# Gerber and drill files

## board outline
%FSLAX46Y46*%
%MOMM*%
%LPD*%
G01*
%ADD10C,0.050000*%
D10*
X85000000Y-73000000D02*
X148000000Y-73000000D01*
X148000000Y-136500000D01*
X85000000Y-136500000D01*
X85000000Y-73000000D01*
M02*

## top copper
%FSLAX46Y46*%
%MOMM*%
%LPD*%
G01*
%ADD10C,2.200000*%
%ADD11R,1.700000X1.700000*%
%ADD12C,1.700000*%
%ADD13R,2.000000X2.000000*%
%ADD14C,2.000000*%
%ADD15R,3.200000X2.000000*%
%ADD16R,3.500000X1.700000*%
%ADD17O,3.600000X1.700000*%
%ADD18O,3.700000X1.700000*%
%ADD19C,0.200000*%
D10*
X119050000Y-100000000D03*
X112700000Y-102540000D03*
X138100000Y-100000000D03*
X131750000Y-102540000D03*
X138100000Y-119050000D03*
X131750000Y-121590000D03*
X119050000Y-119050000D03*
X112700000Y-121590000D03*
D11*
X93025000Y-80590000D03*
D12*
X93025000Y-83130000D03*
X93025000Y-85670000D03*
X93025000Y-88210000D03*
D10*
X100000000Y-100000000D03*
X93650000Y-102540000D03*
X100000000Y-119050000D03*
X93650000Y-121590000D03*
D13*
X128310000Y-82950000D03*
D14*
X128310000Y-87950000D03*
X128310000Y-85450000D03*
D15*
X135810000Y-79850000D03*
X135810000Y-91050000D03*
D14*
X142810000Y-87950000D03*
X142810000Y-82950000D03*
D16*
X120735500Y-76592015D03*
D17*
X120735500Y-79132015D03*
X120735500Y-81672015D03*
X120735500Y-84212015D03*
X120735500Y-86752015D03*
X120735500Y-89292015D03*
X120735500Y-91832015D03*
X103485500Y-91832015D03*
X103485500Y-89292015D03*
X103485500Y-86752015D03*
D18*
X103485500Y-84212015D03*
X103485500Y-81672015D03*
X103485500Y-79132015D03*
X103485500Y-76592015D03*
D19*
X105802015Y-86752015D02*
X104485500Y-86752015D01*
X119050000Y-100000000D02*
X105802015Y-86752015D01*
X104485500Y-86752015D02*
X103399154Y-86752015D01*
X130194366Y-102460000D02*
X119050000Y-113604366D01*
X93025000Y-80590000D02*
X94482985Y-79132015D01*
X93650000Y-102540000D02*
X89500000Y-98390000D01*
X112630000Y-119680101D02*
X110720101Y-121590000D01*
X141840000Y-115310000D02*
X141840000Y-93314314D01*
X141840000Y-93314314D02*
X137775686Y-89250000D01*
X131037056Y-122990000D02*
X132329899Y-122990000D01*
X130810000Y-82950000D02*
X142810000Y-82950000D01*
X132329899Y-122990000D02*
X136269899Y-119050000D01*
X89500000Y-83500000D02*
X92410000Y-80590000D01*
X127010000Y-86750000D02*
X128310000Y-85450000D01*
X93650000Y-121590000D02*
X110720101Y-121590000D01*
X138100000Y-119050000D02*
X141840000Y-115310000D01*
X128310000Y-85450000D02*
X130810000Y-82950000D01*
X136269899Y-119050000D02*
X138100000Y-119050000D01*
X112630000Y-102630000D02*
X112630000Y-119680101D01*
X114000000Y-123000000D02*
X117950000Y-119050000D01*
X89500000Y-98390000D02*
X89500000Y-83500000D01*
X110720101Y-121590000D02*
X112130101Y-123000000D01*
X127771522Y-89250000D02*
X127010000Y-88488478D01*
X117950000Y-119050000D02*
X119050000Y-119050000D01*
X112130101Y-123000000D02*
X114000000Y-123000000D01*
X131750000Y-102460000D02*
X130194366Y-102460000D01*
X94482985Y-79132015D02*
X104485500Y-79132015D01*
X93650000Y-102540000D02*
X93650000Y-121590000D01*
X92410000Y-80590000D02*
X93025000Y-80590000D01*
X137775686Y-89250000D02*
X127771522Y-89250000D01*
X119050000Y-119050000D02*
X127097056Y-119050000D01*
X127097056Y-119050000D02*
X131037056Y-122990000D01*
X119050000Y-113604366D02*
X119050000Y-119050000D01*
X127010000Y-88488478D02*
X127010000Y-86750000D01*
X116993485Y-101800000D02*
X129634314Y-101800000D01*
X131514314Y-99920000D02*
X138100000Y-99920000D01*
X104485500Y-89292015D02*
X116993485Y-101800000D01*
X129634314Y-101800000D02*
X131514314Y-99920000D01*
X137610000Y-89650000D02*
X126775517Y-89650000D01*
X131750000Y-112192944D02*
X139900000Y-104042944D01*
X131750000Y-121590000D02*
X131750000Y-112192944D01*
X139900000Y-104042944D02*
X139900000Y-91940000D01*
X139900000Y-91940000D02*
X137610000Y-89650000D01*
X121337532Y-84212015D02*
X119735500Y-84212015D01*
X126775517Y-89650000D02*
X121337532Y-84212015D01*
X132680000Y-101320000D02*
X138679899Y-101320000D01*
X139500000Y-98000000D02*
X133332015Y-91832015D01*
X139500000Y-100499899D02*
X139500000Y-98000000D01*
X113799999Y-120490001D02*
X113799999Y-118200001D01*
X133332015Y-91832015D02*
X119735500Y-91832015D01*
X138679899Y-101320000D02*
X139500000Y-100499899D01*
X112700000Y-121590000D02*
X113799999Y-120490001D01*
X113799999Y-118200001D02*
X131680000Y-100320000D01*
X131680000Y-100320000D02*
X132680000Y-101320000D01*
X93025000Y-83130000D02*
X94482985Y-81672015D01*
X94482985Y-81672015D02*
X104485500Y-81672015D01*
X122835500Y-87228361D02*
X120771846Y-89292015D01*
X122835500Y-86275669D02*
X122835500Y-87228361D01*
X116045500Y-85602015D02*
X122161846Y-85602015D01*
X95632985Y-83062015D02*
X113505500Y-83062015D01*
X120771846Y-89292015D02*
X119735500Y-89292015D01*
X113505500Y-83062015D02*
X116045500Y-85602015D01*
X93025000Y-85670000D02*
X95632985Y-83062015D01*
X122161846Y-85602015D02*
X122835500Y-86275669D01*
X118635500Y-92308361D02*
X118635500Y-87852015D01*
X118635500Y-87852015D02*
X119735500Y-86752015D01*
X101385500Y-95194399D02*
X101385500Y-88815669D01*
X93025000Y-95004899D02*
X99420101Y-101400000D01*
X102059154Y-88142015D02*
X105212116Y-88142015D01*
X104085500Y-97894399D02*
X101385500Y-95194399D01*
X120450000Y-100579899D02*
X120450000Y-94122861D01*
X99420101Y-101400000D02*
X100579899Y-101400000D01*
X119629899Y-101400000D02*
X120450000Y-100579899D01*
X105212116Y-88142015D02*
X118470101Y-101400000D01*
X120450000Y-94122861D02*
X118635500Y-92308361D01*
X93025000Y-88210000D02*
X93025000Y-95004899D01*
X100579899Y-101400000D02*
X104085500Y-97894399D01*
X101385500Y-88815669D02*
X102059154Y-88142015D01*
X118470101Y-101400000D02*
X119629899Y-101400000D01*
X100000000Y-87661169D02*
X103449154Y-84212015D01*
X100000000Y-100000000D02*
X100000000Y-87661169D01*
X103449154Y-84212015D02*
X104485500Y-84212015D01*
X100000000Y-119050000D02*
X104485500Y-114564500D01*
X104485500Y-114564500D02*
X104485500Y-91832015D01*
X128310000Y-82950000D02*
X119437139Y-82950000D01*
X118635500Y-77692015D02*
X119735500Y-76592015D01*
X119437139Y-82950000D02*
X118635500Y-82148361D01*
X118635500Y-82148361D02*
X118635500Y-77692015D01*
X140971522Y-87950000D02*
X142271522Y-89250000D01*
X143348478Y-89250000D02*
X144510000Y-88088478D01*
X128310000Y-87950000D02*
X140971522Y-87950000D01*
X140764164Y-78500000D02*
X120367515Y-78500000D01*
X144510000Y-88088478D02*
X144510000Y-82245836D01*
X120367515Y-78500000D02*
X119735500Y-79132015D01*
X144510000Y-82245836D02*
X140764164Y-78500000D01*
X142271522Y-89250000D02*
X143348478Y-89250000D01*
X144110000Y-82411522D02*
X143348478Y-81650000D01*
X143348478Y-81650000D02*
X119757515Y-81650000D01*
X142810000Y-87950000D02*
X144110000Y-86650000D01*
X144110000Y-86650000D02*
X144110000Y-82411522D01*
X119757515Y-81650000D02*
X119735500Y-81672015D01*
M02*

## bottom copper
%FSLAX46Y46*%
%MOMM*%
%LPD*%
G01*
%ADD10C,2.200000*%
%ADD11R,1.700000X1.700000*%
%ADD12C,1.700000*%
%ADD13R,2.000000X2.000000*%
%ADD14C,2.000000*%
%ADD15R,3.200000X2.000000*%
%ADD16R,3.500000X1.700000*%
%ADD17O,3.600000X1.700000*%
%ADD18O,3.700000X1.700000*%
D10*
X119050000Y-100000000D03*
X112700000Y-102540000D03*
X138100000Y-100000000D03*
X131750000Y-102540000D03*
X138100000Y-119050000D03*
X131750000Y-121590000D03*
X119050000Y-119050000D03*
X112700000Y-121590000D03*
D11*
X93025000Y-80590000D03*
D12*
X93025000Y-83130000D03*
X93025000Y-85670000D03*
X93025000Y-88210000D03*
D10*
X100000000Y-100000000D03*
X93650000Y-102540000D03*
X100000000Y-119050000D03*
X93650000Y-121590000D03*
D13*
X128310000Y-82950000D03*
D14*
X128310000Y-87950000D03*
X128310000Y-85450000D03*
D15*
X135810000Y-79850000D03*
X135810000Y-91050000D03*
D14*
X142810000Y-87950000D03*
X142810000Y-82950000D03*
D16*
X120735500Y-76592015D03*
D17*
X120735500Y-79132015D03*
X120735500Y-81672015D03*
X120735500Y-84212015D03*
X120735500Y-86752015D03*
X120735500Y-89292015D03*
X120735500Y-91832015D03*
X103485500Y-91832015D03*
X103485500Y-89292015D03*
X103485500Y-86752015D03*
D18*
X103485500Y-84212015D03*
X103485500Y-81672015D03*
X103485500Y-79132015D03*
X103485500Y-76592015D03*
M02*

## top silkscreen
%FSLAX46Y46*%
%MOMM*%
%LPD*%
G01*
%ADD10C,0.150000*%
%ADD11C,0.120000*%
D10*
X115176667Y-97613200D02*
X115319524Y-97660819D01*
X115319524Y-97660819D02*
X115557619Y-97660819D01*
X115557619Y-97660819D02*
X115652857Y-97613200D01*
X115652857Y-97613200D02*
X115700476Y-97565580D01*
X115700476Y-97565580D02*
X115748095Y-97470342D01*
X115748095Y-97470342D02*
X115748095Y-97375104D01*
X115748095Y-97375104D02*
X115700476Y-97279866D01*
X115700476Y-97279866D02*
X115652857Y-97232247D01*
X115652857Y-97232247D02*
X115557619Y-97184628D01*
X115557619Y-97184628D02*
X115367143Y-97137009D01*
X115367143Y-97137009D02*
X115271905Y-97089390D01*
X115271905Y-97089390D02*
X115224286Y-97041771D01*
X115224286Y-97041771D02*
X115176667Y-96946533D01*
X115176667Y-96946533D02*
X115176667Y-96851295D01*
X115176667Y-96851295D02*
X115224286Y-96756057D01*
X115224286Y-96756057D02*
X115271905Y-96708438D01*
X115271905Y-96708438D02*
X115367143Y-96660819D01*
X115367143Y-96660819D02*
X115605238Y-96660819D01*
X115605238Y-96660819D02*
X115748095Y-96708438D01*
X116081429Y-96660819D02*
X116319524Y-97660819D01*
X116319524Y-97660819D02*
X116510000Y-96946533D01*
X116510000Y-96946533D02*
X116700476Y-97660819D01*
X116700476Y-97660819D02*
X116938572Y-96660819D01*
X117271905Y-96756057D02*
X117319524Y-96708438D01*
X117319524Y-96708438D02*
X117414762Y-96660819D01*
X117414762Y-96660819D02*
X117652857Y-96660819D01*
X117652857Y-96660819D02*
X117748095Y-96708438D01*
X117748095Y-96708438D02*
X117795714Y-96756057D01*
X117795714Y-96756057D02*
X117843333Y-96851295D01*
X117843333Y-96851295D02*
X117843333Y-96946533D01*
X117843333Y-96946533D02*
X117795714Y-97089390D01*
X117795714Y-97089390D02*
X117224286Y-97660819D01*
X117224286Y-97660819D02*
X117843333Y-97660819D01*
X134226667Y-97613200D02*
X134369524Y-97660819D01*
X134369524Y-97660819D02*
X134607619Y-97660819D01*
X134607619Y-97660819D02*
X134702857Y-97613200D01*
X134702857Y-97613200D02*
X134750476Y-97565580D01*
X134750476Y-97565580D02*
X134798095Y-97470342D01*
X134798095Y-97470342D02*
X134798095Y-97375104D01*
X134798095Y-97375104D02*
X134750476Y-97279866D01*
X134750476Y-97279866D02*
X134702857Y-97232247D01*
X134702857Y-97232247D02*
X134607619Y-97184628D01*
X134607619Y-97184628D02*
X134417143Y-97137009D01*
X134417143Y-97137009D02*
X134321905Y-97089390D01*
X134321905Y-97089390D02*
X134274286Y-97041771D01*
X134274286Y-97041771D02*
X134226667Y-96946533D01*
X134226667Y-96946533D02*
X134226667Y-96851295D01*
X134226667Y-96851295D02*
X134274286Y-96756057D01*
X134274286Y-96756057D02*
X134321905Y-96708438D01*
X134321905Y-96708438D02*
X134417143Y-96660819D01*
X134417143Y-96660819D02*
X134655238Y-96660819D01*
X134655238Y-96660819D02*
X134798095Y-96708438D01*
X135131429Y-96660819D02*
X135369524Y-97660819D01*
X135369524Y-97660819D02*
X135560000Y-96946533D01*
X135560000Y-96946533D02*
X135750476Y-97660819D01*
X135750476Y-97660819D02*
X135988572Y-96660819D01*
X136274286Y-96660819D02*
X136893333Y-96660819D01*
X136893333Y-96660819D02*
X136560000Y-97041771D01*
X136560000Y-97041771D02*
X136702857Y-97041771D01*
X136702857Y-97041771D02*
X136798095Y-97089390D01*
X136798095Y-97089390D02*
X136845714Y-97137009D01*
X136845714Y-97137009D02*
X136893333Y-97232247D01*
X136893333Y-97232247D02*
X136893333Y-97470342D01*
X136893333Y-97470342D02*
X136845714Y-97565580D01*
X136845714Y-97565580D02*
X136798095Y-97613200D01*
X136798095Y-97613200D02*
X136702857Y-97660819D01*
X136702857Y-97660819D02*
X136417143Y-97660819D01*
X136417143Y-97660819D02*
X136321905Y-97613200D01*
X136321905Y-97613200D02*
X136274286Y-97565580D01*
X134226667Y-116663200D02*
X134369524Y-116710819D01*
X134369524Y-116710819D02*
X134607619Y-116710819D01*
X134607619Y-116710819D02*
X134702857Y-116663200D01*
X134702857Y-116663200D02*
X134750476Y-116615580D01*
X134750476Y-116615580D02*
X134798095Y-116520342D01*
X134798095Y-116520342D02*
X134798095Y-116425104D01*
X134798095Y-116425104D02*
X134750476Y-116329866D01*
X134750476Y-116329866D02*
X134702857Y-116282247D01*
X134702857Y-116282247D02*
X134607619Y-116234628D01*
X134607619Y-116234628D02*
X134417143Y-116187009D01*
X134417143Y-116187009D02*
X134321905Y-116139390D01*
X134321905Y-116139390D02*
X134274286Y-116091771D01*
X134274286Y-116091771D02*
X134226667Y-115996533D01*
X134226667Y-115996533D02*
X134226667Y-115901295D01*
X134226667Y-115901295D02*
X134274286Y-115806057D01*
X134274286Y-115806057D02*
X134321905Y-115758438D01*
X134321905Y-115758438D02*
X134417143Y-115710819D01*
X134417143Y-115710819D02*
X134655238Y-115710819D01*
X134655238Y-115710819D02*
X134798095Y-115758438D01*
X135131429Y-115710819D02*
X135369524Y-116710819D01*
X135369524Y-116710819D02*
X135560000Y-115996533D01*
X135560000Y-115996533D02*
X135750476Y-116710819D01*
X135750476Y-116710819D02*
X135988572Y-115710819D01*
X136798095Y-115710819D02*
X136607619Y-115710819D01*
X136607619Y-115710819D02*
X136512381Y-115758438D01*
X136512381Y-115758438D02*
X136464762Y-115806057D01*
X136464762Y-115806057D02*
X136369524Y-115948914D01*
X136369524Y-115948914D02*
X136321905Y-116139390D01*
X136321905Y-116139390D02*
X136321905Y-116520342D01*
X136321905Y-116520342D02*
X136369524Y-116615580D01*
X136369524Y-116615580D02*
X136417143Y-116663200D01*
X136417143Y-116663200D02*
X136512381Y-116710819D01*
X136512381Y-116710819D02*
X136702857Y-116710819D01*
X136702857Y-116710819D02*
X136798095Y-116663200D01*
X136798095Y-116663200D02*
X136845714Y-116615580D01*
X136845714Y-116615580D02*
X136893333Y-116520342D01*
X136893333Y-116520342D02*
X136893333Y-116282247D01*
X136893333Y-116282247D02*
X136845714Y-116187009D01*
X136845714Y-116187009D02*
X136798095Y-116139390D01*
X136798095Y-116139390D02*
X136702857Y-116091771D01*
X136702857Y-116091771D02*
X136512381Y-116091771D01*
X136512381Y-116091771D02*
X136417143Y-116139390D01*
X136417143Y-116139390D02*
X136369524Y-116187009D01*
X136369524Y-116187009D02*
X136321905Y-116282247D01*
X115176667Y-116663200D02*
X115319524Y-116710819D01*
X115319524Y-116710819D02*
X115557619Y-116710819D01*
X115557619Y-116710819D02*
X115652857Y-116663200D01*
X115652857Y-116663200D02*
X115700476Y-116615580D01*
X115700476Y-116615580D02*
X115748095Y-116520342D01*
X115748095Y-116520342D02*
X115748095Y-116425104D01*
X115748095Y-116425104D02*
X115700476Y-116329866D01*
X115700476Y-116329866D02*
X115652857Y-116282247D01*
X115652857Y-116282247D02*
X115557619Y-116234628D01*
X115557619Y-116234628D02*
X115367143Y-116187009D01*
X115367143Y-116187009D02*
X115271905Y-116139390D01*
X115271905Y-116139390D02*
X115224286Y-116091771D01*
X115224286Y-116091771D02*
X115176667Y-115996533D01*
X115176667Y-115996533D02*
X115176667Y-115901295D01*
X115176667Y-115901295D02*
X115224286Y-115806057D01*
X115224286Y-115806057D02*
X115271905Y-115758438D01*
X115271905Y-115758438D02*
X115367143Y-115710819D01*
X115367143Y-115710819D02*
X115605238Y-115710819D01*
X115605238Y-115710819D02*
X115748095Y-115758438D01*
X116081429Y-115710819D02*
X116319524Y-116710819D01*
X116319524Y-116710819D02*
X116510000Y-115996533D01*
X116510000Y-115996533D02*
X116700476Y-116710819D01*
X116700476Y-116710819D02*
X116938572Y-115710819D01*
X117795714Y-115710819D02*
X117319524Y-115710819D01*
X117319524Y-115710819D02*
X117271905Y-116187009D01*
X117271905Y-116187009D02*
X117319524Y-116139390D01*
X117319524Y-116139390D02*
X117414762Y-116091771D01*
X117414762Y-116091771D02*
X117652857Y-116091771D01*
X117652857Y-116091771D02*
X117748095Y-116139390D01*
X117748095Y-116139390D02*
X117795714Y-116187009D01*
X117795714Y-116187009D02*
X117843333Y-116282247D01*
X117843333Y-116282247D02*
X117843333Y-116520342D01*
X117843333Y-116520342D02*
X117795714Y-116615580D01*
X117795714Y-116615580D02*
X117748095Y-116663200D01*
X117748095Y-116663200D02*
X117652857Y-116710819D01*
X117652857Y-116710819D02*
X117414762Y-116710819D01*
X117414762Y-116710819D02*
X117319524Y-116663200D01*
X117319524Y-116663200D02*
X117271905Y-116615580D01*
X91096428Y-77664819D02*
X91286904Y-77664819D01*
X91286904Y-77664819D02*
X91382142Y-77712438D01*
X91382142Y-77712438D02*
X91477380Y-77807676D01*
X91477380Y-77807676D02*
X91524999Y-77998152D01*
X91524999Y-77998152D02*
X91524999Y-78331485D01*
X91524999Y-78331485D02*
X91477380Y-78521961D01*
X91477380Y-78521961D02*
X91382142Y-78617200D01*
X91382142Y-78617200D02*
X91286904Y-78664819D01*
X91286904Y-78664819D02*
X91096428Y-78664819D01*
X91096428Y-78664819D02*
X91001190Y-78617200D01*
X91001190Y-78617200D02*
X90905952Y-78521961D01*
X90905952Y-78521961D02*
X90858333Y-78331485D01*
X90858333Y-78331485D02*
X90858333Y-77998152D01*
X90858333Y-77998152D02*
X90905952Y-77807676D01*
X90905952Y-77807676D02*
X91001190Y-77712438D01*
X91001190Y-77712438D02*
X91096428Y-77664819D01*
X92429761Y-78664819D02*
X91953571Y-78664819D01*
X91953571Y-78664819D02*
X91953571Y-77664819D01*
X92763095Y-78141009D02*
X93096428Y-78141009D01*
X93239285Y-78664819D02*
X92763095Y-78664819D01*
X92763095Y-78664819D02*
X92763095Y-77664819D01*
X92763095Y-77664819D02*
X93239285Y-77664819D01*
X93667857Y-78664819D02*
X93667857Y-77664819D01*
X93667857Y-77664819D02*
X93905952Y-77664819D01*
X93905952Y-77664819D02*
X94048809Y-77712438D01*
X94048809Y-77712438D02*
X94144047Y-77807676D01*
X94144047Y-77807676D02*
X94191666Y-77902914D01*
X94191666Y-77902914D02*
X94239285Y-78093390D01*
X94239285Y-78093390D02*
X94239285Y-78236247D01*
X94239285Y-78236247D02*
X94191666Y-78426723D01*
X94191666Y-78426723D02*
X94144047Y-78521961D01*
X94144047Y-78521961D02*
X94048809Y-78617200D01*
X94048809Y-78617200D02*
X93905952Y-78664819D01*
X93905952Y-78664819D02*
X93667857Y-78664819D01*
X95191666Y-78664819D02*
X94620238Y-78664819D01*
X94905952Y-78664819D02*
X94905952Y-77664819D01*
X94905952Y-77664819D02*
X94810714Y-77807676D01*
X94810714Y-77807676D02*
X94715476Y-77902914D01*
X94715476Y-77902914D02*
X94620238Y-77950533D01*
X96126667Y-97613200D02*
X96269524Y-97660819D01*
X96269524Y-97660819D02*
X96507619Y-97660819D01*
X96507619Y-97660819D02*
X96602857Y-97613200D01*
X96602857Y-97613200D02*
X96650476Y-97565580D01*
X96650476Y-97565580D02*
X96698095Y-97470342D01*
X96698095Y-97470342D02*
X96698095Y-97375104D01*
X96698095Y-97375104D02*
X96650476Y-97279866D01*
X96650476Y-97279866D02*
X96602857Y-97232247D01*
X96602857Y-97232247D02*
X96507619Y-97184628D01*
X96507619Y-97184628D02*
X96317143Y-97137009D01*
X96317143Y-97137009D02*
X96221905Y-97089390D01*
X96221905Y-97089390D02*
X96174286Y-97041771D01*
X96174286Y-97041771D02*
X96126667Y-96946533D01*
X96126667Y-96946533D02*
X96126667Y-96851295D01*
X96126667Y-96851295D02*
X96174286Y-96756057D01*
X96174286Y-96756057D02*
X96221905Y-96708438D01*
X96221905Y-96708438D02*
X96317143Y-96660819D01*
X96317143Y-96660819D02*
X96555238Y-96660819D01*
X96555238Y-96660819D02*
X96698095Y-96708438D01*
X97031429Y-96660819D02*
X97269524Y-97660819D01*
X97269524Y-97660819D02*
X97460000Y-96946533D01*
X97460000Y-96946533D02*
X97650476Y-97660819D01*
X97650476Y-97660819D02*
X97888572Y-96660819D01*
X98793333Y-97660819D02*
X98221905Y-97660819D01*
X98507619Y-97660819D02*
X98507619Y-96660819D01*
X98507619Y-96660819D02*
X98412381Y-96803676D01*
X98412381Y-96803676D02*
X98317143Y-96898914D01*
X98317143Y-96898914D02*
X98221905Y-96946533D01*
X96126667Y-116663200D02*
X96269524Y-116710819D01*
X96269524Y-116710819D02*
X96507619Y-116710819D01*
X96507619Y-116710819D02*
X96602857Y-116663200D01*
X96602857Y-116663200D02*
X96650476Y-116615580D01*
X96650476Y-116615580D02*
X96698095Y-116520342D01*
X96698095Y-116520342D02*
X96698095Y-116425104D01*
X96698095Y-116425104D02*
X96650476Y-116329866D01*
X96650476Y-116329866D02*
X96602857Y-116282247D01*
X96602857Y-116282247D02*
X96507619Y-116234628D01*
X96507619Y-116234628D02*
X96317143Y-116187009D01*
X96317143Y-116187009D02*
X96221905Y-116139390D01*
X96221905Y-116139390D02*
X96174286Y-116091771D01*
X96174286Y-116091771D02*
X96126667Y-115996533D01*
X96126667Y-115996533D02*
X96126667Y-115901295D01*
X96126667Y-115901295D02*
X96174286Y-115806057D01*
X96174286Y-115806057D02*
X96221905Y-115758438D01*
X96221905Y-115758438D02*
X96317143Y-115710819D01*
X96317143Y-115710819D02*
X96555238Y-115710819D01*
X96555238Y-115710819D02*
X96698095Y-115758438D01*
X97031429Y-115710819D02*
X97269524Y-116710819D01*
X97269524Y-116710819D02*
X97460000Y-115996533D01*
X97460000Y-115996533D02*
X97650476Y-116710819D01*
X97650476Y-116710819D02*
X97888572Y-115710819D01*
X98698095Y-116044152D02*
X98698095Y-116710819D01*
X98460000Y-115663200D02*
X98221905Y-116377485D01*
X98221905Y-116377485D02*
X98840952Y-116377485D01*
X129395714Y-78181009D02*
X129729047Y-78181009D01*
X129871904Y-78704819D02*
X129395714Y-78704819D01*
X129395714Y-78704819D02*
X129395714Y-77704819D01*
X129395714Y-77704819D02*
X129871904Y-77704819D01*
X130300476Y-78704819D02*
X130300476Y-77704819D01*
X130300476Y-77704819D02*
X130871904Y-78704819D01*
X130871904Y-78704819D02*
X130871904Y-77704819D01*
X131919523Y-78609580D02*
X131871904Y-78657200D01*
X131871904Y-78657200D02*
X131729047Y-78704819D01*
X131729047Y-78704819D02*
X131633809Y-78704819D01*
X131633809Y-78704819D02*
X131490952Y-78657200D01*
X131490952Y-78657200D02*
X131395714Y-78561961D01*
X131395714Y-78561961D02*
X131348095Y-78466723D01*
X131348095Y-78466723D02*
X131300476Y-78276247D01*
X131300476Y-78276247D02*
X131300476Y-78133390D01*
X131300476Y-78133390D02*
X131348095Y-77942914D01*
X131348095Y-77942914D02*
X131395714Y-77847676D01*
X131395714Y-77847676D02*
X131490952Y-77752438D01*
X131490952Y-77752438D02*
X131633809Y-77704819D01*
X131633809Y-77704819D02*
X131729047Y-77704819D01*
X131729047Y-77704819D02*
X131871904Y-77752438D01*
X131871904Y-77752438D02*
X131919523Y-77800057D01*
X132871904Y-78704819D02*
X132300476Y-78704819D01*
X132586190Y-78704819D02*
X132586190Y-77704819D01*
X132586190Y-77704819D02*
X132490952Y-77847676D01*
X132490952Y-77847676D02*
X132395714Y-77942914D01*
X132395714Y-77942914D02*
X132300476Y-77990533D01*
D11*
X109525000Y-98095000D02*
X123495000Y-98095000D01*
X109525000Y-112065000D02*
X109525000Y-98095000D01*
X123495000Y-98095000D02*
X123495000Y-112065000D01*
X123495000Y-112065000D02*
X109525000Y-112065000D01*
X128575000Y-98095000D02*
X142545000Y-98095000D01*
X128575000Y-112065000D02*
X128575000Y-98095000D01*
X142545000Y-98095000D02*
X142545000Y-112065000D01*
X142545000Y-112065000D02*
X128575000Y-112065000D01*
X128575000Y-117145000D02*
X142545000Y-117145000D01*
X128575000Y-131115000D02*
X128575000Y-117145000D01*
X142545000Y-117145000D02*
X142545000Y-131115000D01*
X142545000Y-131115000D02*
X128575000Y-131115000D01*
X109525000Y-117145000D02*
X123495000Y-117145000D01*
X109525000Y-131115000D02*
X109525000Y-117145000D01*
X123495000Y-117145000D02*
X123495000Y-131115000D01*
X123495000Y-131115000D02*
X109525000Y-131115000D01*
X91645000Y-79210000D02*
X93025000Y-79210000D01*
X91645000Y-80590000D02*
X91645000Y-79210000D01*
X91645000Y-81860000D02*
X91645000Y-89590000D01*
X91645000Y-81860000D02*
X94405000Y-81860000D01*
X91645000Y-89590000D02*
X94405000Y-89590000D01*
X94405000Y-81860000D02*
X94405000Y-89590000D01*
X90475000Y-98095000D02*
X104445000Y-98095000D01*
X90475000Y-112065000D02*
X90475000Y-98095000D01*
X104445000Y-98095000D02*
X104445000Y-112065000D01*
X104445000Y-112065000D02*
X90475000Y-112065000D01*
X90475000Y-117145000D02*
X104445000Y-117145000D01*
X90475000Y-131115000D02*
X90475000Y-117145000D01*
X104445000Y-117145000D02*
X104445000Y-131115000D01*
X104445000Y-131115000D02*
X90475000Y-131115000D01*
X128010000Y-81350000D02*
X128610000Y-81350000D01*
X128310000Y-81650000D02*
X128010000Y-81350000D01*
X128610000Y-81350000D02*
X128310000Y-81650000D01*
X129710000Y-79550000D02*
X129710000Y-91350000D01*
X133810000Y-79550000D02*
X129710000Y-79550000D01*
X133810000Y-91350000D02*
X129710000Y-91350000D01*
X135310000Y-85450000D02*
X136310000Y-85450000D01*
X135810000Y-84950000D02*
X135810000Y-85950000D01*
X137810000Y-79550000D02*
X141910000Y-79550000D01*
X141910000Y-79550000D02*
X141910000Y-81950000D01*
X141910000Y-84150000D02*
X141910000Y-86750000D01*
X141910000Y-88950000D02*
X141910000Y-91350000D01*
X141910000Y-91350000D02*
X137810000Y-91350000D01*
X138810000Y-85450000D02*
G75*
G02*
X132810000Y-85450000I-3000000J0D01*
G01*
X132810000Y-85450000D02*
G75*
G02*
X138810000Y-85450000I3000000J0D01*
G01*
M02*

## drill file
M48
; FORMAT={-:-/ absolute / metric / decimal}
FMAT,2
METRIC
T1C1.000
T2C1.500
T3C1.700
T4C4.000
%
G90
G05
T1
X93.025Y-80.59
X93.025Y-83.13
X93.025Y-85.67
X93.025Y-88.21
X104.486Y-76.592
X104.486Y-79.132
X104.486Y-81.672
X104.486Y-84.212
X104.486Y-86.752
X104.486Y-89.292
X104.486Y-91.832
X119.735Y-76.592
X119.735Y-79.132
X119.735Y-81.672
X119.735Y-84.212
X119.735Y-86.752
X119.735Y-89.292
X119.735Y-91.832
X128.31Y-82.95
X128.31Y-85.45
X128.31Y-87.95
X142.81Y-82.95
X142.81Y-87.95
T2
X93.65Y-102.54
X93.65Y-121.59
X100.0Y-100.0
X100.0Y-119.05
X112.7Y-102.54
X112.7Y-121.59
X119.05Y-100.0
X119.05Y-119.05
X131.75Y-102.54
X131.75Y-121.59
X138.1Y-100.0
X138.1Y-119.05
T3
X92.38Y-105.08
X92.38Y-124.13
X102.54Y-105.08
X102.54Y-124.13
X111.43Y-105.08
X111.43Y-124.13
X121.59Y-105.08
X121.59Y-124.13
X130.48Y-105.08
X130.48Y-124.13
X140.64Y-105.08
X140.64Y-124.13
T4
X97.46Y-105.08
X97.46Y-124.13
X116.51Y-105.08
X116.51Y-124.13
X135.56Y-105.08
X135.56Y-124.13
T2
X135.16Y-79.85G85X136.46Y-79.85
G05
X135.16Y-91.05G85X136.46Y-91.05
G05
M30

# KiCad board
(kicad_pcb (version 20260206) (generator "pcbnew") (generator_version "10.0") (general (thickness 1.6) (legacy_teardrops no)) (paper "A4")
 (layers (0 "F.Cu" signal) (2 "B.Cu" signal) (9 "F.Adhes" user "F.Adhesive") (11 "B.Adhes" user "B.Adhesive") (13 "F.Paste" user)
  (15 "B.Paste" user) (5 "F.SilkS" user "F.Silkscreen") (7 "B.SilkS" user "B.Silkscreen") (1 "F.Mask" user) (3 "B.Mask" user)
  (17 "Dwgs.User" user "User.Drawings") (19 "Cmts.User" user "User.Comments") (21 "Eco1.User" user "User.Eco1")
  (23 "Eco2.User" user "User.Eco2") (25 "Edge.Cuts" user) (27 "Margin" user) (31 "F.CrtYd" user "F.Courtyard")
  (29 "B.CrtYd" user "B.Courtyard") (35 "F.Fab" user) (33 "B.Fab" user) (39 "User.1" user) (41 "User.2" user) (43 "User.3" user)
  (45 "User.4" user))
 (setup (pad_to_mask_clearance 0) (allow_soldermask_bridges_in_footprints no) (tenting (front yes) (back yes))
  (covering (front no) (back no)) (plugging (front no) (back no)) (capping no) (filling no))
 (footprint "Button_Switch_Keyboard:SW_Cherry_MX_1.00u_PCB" (layer "F.Cu") (at 119.05 100)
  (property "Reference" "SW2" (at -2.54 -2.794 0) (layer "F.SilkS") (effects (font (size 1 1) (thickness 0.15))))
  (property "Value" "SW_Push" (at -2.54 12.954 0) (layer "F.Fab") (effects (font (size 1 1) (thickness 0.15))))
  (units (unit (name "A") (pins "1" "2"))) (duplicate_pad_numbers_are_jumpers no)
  (fp_line (start -9.525 -1.905) (end 4.445 -1.905) (stroke (width 0.12) (type solid)) (layer "F.SilkS"))
  (fp_line (start -9.525 12.065) (end -9.525 -1.905) (stroke (width 0.12) (type solid)) (layer "F.SilkS"))
  (fp_line (start 4.445 -1.905) (end 4.445 12.065) (stroke (width 0.12) (type solid)) (layer "F.SilkS"))
  (fp_line (start 4.445 12.065) (end -9.525 12.065) (stroke (width 0.12) (type solid)) (layer "F.SilkS"))
  (pad "" np_thru_hole circle (at -7.62 5.08) (size 1.7 1.7) (drill 1.7) (layers "*.Cu" "*.Mask"))
  (pad "" np_thru_hole circle (at -2.54 5.08) (size 4 4) (drill 4) (layers "*.Cu" "*.Mask"))
  (pad "" np_thru_hole circle (at 2.54 5.08) (size 1.7 1.7) (drill 1.7) (layers "*.Cu" "*.Mask"))
  (pad "1" thru_hole circle (at 0 0) (size 2.2 2.2) (drill 1.5) (layers "*.Cu" "*.Mask") (remove_unused_layers no)
   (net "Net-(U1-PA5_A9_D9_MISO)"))
  (pad "2" thru_hole circle (at -6.35 2.54) (size 2.2 2.2) (drill 1.5) (layers "*.Cu" "*.Mask") (remove_unused_layers no) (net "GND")))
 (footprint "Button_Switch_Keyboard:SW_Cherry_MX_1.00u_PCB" (layer "F.Cu") (at 138.1 100)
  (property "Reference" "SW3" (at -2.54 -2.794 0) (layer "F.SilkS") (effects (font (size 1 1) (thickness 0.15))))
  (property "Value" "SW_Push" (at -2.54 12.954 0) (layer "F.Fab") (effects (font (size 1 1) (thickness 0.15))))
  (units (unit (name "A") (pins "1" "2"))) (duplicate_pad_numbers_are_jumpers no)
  (fp_line (start -9.525 -1.905) (end 4.445 -1.905) (stroke (width 0.12) (type solid)) (layer "F.SilkS"))
  (fp_line (start -9.525 12.065) (end -9.525 -1.905) (stroke (width 0.12) (type solid)) (layer "F.SilkS"))
  (fp_line (start 4.445 -1.905) (end 4.445 12.065) (stroke (width 0.12) (type solid)) (layer "F.SilkS"))
  (fp_line (start 4.445 12.065) (end -9.525 12.065) (stroke (width 0.12) (type solid)) (layer "F.SilkS"))
  (pad "" np_thru_hole circle (at -7.62 5.08) (size 1.7 1.7) (drill 1.7) (layers "*.Cu" "*.Mask"))
  (pad "" np_thru_hole circle (at -2.54 5.08) (size 4 4) (drill 4) (layers "*.Cu" "*.Mask"))
  (pad "" np_thru_hole circle (at 2.54 5.08) (size 1.7 1.7) (drill 1.7) (layers "*.Cu" "*.Mask"))
  (pad "1" thru_hole circle (at 0 0) (size 2.2 2.2) (drill 1.5) (layers "*.Cu" "*.Mask") (remove_unused_layers no)
   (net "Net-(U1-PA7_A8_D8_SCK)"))
  (pad "2" thru_hole circle (at -6.35 2.54) (size 2.2 2.2) (drill 1.5) (layers "*.Cu" "*.Mask") (remove_unused_layers no) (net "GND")))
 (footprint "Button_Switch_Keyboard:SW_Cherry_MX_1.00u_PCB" (layer "F.Cu") (at 138.1 119.05)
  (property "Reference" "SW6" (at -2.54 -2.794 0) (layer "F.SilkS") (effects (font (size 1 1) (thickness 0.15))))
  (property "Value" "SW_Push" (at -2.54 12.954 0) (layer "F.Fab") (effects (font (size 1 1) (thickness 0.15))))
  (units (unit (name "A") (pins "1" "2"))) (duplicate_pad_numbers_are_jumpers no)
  (fp_line (start -9.525 -1.905) (end 4.445 -1.905) (stroke (width 0.12) (type solid)) (layer "F.SilkS"))
  (fp_line (start -9.525 12.065) (end -9.525 -1.905) (stroke (width 0.12) (type solid)) (layer "F.SilkS"))
  (fp_line (start 4.445 -1.905) (end 4.445 12.065) (stroke (width 0.12) (type solid)) (layer "F.SilkS"))
  (fp_line (start 4.445 12.065) (end -9.525 12.065) (stroke (width 0.12) (type solid)) (layer "F.SilkS"))
  (pad "" np_thru_hole circle (at -7.62 5.08) (size 1.7 1.7) (drill 1.7) (layers "*.Cu" "*.Mask"))
  (pad "" np_thru_hole circle (at -2.54 5.08) (size 4 4) (drill 4) (layers "*.Cu" "*.Mask"))
  (pad "" np_thru_hole circle (at 2.54 5.08) (size 1.7 1.7) (drill 1.7) (layers "*.Cu" "*.Mask"))
  (pad "1" thru_hole circle (at 0 0) (size 2.2 2.2) (drill 1.5) (layers "*.Cu" "*.Mask") (remove_unused_layers no) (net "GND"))
  (pad "2" thru_hole circle (at -6.35 2.54) (size 2.2 2.2) (drill 1.5) (layers "*.Cu" "*.Mask") (remove_unused_layers no)
   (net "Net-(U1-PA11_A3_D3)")))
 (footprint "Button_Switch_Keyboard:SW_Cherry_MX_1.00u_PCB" (layer "F.Cu") (at 119.05 119.05)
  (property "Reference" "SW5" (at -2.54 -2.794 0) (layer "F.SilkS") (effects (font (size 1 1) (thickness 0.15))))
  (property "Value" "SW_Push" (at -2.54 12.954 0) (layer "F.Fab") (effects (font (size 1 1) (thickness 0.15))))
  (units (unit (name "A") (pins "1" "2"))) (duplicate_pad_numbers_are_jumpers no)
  (fp_line (start -9.525 -1.905) (end 4.445 -1.905) (stroke (width 0.12) (type solid)) (layer "F.SilkS"))
  (fp_line (start -9.525 12.065) (end -9.525 -1.905) (stroke (width 0.12) (type solid)) (layer "F.SilkS"))
  (fp_line (start 4.445 -1.905) (end 4.445 12.065) (stroke (width 0.12) (type solid)) (layer "F.SilkS"))
  (fp_line (start 4.445 12.065) (end -9.525 12.065) (stroke (width 0.12) (type solid)) (layer "F.SilkS"))
  (pad "" np_thru_hole circle (at -7.62 5.08) (size 1.7 1.7) (drill 1.7) (layers "*.Cu" "*.Mask"))
  (pad "" np_thru_hole circle (at -2.54 5.08) (size 4 4) (drill 4) (layers "*.Cu" "*.Mask"))
  (pad "" np_thru_hole circle (at 2.54 5.08) (size 1.7 1.7) (drill 1.7) (layers "*.Cu" "*.Mask"))
  (pad "1" thru_hole circle (at 0 0) (size 2.2 2.2) (drill 1.5) (layers "*.Cu" "*.Mask") (remove_unused_layers no) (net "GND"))
  (pad "2" thru_hole circle (at -6.35 2.54) (size 2.2 2.2) (drill 1.5) (layers "*.Cu" "*.Mask") (remove_unused_layers no)
   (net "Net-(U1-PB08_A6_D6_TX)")))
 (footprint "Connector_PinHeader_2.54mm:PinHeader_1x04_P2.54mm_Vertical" (layer "F.Cu") (at 93.025 80.59)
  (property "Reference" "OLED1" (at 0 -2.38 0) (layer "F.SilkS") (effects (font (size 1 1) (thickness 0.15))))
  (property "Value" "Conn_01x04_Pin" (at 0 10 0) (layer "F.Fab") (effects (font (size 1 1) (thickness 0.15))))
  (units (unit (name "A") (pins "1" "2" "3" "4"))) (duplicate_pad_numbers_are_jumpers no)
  (fp_line (start -1.38 -1.38) (end 0 -1.38) (stroke (width 0.12) (type solid)) (layer "F.SilkS"))
  (fp_line (start -1.38 0) (end -1.38 -1.38) (stroke (width 0.12) (type solid)) (layer "F.SilkS"))
  (fp_line (start -1.38 1.27) (end -1.38 9) (stroke (width 0.12) (type solid)) (layer "F.SilkS"))
  (fp_line (start -1.38 1.27) (end 1.38 1.27) (stroke (width 0.12) (type solid)) (layer "F.SilkS"))
  (fp_line (start -1.38 9) (end 1.38 9) (stroke (width 0.12) (type solid)) (layer "F.SilkS"))
  (fp_line (start 1.38 1.27) (end 1.38 9) (stroke (width 0.12) (type solid)) (layer "F.SilkS"))
  (pad "1" thru_hole rect (at 0 0) (size 1.7 1.7) (drill 1) (layers "*.Cu" "*.Mask") (remove_unused_layers no) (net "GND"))
  (pad "2" thru_hole circle (at 0 2.54) (size 1.7 1.7) (drill 1) (layers "*.Cu" "*.Mask") (remove_unused_layers no) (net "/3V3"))
  (pad "3" thru_hole circle (at 0 5.08) (size 1.7 1.7) (drill 1) (layers "*.Cu" "*.Mask") (remove_unused_layers no) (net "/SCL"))
  (pad "4" thru_hole circle (at 0 7.62) (size 1.7 1.7) (drill 1) (layers "*.Cu" "*.Mask") (remove_unused_layers no) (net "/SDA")))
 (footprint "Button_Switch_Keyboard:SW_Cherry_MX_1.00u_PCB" (layer "F.Cu") (at 100 100)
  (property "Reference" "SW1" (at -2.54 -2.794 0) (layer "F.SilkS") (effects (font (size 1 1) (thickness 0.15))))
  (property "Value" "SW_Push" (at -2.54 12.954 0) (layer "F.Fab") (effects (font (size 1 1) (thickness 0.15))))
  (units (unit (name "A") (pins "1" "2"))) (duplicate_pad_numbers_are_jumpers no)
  (fp_line (start -9.525 -1.905) (end 4.445 -1.905) (stroke (width 0.12) (type solid)) (layer "F.SilkS"))
  (fp_line (start -9.525 12.065) (end -9.525 -1.905) (stroke (width 0.12) (type solid)) (layer "F.SilkS"))
  (fp_line (start 4.445 -1.905) (end 4.445 12.065) (stroke (width 0.12) (type solid)) (layer "F.SilkS"))
  (fp_line (start 4.445 12.065) (end -9.525 12.065) (stroke (width 0.12) (type solid)) (layer "F.SilkS"))
  (pad "" np_thru_hole circle (at -7.62 5.08) (size 1.7 1.7) (drill 1.7) (layers "*.Cu" "*.Mask"))
  (pad "" np_thru_hole circle (at -2.54 5.08) (size 4 4) (drill 4) (layers "*.Cu" "*.Mask"))
  (pad "" np_thru_hole circle (at 2.54 5.08) (size 1.7 1.7) (drill 1.7) (layers "*.Cu" "*.Mask"))
  (pad "1" thru_hole circle (at 0 0) (size 2.2 2.2) (drill 1.5) (layers "*.Cu" "*.Mask") (remove_unused_layers no)
   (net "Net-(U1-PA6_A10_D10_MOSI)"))
  (pad "2" thru_hole circle (at -6.35 2.54) (size 2.2 2.2) (drill 1.5) (layers "*.Cu" "*.Mask") (remove_unused_layers no) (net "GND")))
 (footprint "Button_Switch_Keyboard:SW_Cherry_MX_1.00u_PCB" (layer "F.Cu") (at 100 119.05)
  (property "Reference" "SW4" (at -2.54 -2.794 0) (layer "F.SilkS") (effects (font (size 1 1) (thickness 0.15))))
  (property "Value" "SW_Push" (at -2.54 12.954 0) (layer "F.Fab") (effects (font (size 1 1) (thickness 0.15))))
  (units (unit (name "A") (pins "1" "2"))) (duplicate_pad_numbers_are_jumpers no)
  (fp_line (start -9.525 -1.905) (end 4.445 -1.905) (stroke (width 0.12) (type solid)) (layer "F.SilkS"))
  (fp_line (start -9.525 12.065) (end -9.525 -1.905) (stroke (width 0.12) (type solid)) (layer "F.SilkS"))
  (fp_line (start 4.445 -1.905) (end 4.445 12.065) (stroke (width 0.12) (type solid)) (layer "F.SilkS"))
  (fp_line (start 4.445 12.065) (end -9.525 12.065) (stroke (width 0.12) (type solid)) (layer "F.SilkS"))
  (pad "" np_thru_hole circle (at -7.62 5.08) (size 1.7 1.7) (drill 1.7) (layers "*.Cu" "*.Mask"))
  (pad "" np_thru_hole circle (at -2.54 5.08) (size 4 4) (drill 4) (layers "*.Cu" "*.Mask"))
  (pad "" np_thru_hole circle (at 2.54 5.08) (size 1.7 1.7) (drill 1.7) (layers "*.Cu" "*.Mask"))
  (pad "1" thru_hole circle (at 0 0) (size 2.2 2.2) (drill 1.5) (layers "*.Cu" "*.Mask") (remove_unused_layers no)
   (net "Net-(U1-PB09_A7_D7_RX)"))
  (pad "2" thru_hole circle (at -6.35 2.54) (size 2.2 2.2) (drill 1.5) (layers "*.Cu" "*.Mask") (remove_unused_layers no) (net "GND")))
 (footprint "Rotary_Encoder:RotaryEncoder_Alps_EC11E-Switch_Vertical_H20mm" (layer "F.Cu") (at 128.31 82.95)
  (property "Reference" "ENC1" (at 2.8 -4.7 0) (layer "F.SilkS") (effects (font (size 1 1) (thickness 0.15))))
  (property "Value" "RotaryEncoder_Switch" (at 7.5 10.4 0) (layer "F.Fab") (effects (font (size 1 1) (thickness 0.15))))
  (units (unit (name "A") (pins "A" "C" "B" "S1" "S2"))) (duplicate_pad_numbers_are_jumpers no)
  (fp_line (start -0.3 -1.6) (end 0.3 -1.6) (stroke (width 0.12) (type solid)) (layer "F.SilkS"))
  (fp_line (start 0 -1.3) (end -0.3 -1.6) (stroke (width 0.12) (type solid)) (layer "F.SilkS"))
  (fp_line (start 0.3 -1.6) (end 0 -1.3) (stroke (width 0.12) (type solid)) (layer "F.SilkS"))
  (fp_line (start 1.4 -3.4) (end 1.4 8.4) (stroke (width 0.12) (type solid)) (layer "F.SilkS"))
  (fp_line (start 5.5 -3.4) (end 1.4 -3.4) (stroke (width 0.12) (type solid)) (layer "F.SilkS"))
  (fp_line (start 5.5 8.4) (end 1.4 8.4) (stroke (width 0.12) (type solid)) (layer "F.SilkS"))
  (fp_line (start 7 2.5) (end 8 2.5) (stroke (width 0.12) (type solid)) (layer "F.SilkS"))
  (fp_line (start 7.5 2) (end 7.5 3) (stroke (width 0.12) (type solid)) (layer "F.SilkS"))
  (fp_line (start 9.5 -3.4) (end 13.6 -3.4) (stroke (width 0.12) (type solid)) (layer "F.SilkS"))
  (fp_line (start 13.6 -3.4) (end 13.6 -1) (stroke (width 0.12) (type solid)) (layer "F.SilkS"))
  (fp_line (start 13.6 1.2) (end 13.6 3.8) (stroke (width 0.12) (type solid)) (layer "F.SilkS"))
  (fp_line (start 13.6 6) (end 13.6 8.4) (stroke (width 0.12) (type solid)) (layer "F.SilkS"))
  (fp_line (start 13.6 8.4) (end 9.5 8.4) (stroke (width 0.12) (type solid)) (layer "F.SilkS"))
  (fp_circle (center 7.5 2.5) (end 10.5 2.5) (stroke (width 0.12) (type solid)) (fill no) (layer "F.SilkS"))
  (pad "A" thru_hole rect (at 0 0) (size 2 2) (drill 1) (layers "*.Cu" "*.Mask") (remove_unused_layers no) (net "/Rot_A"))
  (pad "B" thru_hole circle (at 0 5) (size 2 2) (drill 1) (layers "*.Cu" "*.Mask") (remove_unused_layers no) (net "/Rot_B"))
  (pad "C" thru_hole circle (at 0 2.5) (size 2 2) (drill 1) (layers "*.Cu" "*.Mask") (remove_unused_layers no) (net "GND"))
  (pad "MP" thru_hole rect (at 7.5 -3.1) (size 3.2 2) (drill oval 2.8 1.5) (layers "*.Cu" "*.Mask") (remove_unused_layers no))
  (pad "MP" thru_hole rect (at 7.5 8.1) (size 3.2 2) (drill oval 2.8 1.5) (layers "*.Cu" "*.Mask") (remove_unused_layers no))
  (pad "S1" thru_hole circle (at 14.5 5) (size 2 2) (drill 1) (layers "*.Cu" "*.Mask") (remove_unused_layers no) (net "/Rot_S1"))
  (pad "S2" thru_hole circle (at 14.5 0) (size 2 2) (drill 1) (layers "*.Cu" "*.Mask") (remove_unused_layers no) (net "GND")))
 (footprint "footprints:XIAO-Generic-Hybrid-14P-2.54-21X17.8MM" (layer "B.Cu") (at 112.1105 84.212015 180)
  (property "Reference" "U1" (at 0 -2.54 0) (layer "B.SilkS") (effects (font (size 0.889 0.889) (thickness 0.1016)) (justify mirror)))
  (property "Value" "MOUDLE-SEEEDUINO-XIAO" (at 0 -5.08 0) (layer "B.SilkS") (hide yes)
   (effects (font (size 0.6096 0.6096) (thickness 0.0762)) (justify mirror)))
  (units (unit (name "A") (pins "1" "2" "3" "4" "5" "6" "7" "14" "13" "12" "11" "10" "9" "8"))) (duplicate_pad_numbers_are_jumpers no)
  (pad "1" thru_hole rect (at -7.625 7.62 180) (size 3.5 1.7) (drill 1 (offset -1 0)) (layers "*.Cu" "*.Mask") (remove_unused_layers no)
   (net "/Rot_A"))
  (pad "2" thru_hole oval (at -7.625 5.08 180) (size 3.6 1.7) (drill 1 (offset -1 0)) (layers "*.Cu" "*.Mask") (remove_unused_layers no)
   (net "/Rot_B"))
  (pad "3" thru_hole oval (at -7.625 2.54 180) (size 3.6 1.7) (drill 1 (offset -1 0)) (layers "*.Cu" "*.Mask") (remove_unused_layers no)
   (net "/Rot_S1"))
  (pad "4" thru_hole oval (at -7.625 0 180) (size 3.6 1.7) (drill 1 (offset -1 0)) (layers "*.Cu" "*.Mask") (remove_unused_layers no)
   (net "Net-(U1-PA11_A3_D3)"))
  (pad "5" thru_hole oval (at -7.625 -2.54 180) (size 3.6 1.7) (drill 1 (offset -1 0)) (layers "*.Cu" "*.Mask") (remove_unused_layers no)
   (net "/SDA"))
  (pad "6" thru_hole oval (at -7.625 -5.08) (size 3.6 1.7) (drill 1 (offset 1 0)) (layers "*.Cu" "*.Mask") (remove_unused_layers no)
   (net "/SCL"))
  (pad "7" thru_hole oval (at -7.625 -7.62 180) (size 3.6 1.7) (drill 1 (offset -1 0)) (layers "*.Cu" "*.Mask") (remove_unused_layers no)
   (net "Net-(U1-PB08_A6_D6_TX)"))
  (pad "8" thru_hole oval (at 7.625 -7.62 180) (size 3.6 1.7) (drill 1 (offset 1 0)) (layers "*.Cu" "*.Mask") (remove_unused_layers no)
   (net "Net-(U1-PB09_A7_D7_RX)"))
  (pad "9" thru_hole oval (at 7.625 -5.08 180) (size 3.6 1.7) (drill 1 (offset 1 0)) (layers "*.Cu" "*.Mask") (remove_unused_layers no)
   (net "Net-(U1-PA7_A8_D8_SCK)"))
  (pad "10" thru_hole oval (at 7.625 -2.54 180) (size 3.6 1.7) (drill 1 (offset 1 0)) (layers "*.Cu" "*.Mask") (remove_unused_layers no)
   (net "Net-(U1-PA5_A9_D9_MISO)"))
  (pad "11" thru_hole oval (at 7.625 0 180) (size 3.7 1.7) (drill 1 (offset 1 0)) (layers "*.Cu" "*.Mask") (remove_unused_layers no)
   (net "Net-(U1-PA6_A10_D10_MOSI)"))
  (pad "12" thru_hole oval (at 7.625 2.54 180) (size 3.7 1.7) (drill 1 (offset 1 0)) (layers "*.Cu" "*.Mask") (remove_unused_layers no)
   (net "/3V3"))
  (pad "13" thru_hole oval (at 7.625 5.08 180) (size 3.7 1.7) (drill 1 (offset 1 0)) (layers "*.Cu" "*.Mask") (remove_unused_layers no)
   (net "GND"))
  (pad "14" thru_hole oval (at 7.625 7.62 180) (size 3.7 1.7) (drill 1 (offset 1 0)) (layers "*.Cu" "*.Mask") (remove_unused_layers no)
   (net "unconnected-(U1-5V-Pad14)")))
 (gr_rect (start 85 73) (end 148 136.5) (stroke (width 0.05) (type default)) (fill no) (layer "Edge.Cuts"))
 (segment (start 105.802015 86.752015) (end 104.4855 86.752015) (width 0.2) (layer "F.Cu") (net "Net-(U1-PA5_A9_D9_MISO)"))
 (segment (start 119.05 100) (end 105.802015 86.752015) (width 0.2) (layer "F.Cu") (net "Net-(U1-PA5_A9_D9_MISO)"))
 (segment (start 104.4855 86.752015) (end 103.399154 86.752015) (width 0.2) (layer "F.Cu") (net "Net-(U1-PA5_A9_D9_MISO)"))
 (segment (start 130.194366 102.46) (end 119.05 113.604366) (width 0.2) (layer "F.Cu") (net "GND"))
 (segment (start 93.025 80.59) (end 94.482985 79.132015) (width 0.2) (layer "F.Cu") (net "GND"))
 (segment (start 93.65 102.54) (end 89.5 98.39) (width 0.2) (layer "F.Cu") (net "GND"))
 (segment (start 112.63 119.680101) (end 110.720101 121.59) (width 0.2) (layer "F.Cu") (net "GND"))
 (segment (start 141.84 115.31) (end 141.84 93.314314) (width 0.2) (layer "F.Cu") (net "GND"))
 (segment (start 141.84 93.314314) (end 137.775686 89.25) (width 0.2) (layer "F.Cu") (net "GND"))
 (segment (start 131.037056 122.99) (end 132.329899 122.99) (width 0.2) (layer "F.Cu") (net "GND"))
 (segment (start 130.81 82.95) (end 142.81 82.95) (width 0.2) (layer "F.Cu") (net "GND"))
 (segment (start 132.329899 122.99) (end 136.269899 119.05) (width 0.2) (layer "F.Cu") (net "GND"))
 (segment (start 89.5 83.5) (end 92.41 80.59) (width 0.2) (layer "F.Cu") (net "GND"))
 (segment (start 127.01 86.75) (end 128.31 85.45) (width 0.2) (layer "F.Cu") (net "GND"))
 (segment (start 93.65 121.59) (end 110.720101 121.59) (width 0.2) (layer "F.Cu") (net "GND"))
 (segment (start 138.1 119.05) (end 141.84 115.31) (width 0.2) (layer "F.Cu") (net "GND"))
 (segment (start 128.31 85.45) (end 130.81 82.95) (width 0.2) (layer "F.Cu") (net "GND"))
 (segment (start 136.269899 119.05) (end 138.1 119.05) (width 0.2) (layer "F.Cu") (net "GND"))
 (segment (start 112.63 102.63) (end 112.63 119.680101) (width 0.2) (layer "F.Cu") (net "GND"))
 (segment (start 114 123) (end 117.95 119.05) (width 0.2) (layer "F.Cu") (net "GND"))
 (segment (start 89.5 98.39) (end 89.5 83.5) (width 0.2) (layer "F.Cu") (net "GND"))
 (segment (start 110.720101 121.59) (end 112.130101 123) (width 0.2) (layer "F.Cu") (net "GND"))
 (segment (start 127.771522 89.25) (end 127.01 88.488478) (width 0.2) (layer "F.Cu") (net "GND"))
 (segment (start 117.95 119.05) (end 119.05 119.05) (width 0.2) (layer "F.Cu") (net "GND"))
 (segment (start 112.130101 123) (end 114 123) (width 0.2) (layer "F.Cu") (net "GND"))
 (segment (start 131.75 102.46) (end 130.194366 102.46) (width 0.2) (layer "F.Cu") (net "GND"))
 (segment (start 94.482985 79.132015) (end 104.4855 79.132015) (width 0.2) (layer "F.Cu") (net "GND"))
 (segment (start 93.65 102.54) (end 93.65 121.59) (width 0.2) (layer "F.Cu") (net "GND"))
 (segment (start 92.41 80.59) (end 93.025 80.59) (width 0.2) (layer "F.Cu") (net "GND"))
 (segment (start 137.775686 89.25) (end 127.771522 89.25) (width 0.2) (layer "F.Cu") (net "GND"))
 (segment (start 119.05 119.05) (end 127.097056 119.05) (width 0.2) (layer "F.Cu") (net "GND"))
 (segment (start 127.097056 119.05) (end 131.037056 122.99) (width 0.2) (layer "F.Cu") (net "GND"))
 (segment (start 119.05 113.604366) (end 119.05 119.05) (width 0.2) (layer "F.Cu") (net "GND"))
 (segment (start 127.01 88.488478) (end 127.01 86.75) (width 0.2) (layer "F.Cu") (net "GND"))
 (segment (start 116.993485 101.8) (end 129.634314 101.8) (width 0.2) (layer "F.Cu") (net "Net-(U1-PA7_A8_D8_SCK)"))
 (segment (start 131.514314 99.92) (end 138.1 99.92) (width 0.2) (layer "F.Cu") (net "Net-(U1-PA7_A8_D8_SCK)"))
 (segment (start 104.4855 89.292015) (end 116.993485 101.8) (width 0.2) (layer "F.Cu") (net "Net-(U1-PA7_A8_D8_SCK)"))
 (segment (start 129.634314 101.8) (end 131.514314 99.92) (width 0.2) (layer "F.Cu") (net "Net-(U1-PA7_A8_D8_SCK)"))
 (segment (start 137.61 89.65) (end 126.775517 89.65) (width 0.2) (layer "F.Cu") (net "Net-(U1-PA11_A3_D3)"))
 (segment (start 131.75 112.192944) (end 139.9 104.042944) (width 0.2) (layer "F.Cu") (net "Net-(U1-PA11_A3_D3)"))
 (segment (start 131.75 121.59) (end 131.75 112.192944) (width 0.2) (layer "F.Cu") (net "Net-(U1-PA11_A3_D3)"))
 (segment (start 139.9 104.042944) (end 139.9 91.94) (width 0.2) (layer "F.Cu") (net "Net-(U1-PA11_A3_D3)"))
 (segment (start 139.9 91.94) (end 137.61 89.65) (width 0.2) (layer "F.Cu") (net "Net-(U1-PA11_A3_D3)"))
 (segment (start 121.337532 84.212015) (end 119.7355 84.212015) (width 0.2) (layer "F.Cu") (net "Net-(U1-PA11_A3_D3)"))
 (segment (start 126.775517 89.65) (end 121.337532 84.212015) (width 0.2) (layer "F.Cu") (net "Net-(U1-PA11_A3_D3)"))
 (segment (start 132.68 101.32) (end 138.679899 101.32) (width 0.2) (layer "F.Cu") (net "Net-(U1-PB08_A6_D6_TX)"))
 (segment (start 139.5 98) (end 133.332015 91.832015) (width 0.2) (layer "F.Cu") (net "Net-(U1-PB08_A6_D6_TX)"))
 (segment (start 139.5 100.499899) (end 139.5 98) (width 0.2) (layer "F.Cu") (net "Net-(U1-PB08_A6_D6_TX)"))
 (segment (start 113.799999 120.490001) (end 113.799999 118.200001) (width 0.2) (layer "F.Cu") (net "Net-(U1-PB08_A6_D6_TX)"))
 (segment (start 133.332015 91.832015) (end 119.7355 91.832015) (width 0.2) (layer "F.Cu") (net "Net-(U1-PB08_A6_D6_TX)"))
 (segment (start 138.679899 101.32) (end 139.5 100.499899) (width 0.2) (layer "F.Cu") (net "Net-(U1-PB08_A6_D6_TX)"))
 (segment (start 112.7 121.59) (end 113.799999 120.490001) (width 0.2) (layer "F.Cu") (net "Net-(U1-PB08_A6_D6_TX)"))
 (segment (start 113.799999 118.200001) (end 131.68 100.32) (width 0.2) (layer "F.Cu") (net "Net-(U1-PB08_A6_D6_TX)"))
 (segment (start 131.68 100.32) (end 132.68 101.32) (width 0.2) (layer "F.Cu") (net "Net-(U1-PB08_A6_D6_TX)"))
 (segment (start 93.025 83.13) (end 94.482985 81.672015) (width 0.2) (layer "F.Cu") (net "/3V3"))
 (segment (start 94.482985 81.672015) (end 104.4855 81.672015) (width 0.2) (layer "F.Cu") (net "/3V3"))
 (segment (start 122.8355 87.228361) (end 120.771846 89.292015) (width 0.2) (layer "F.Cu") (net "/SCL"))
 (segment (start 122.8355 86.275669) (end 122.8355 87.228361) (width 0.2) (layer "F.Cu") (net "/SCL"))
 (segment (start 116.0455 85.602015) (end 122.161846 85.602015) (width 0.2) (layer "F.Cu") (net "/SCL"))
 (segment (start 95.632985 83.062015) (end 113.5055 83.062015) (width 0.2) (layer "F.Cu") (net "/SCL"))
 (segment (start 120.771846 89.292015) (end 119.7355 89.292015) (width 0.2) (layer "F.Cu") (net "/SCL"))
 (segment (start 113.5055 83.062015) (end 116.0455 85.602015) (width 0.2) (layer "F.Cu") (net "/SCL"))
 (segment (start 93.025 85.67) (end 95.632985 83.062015) (width 0.2) (layer "F.Cu") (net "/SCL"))
 (segment (start 122.161846 85.602015) (end 122.8355 86.275669) (width 0.2) (layer "F.Cu") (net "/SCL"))
 (segment (start 118.6355 92.308361) (end 118.6355 87.852015) (width 0.2) (layer "F.Cu") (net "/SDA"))
 (segment (start 118.6355 87.852015) (end 119.7355 86.752015) (width 0.2) (layer "F.Cu") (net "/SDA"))
 (segment (start 101.3855 95.194399) (end 101.3855 88.815669) (width 0.2) (layer "F.Cu") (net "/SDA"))
 (segment (start 93.025 95.004899) (end 99.420101 101.4) (width 0.2) (layer "F.Cu") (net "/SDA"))
 (segment (start 102.059154 88.142015) (end 105.212116 88.142015) (width 0.2) (layer "F.Cu") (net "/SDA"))
 (segment (start 104.0855 97.894399) (end 101.3855 95.194399) (width 0.2) (layer "F.Cu") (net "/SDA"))
 (segment (start 120.45 100.579899) (end 120.45 94.122861) (width 0.2) (layer "F.Cu") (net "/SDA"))
 (segment (start 99.420101 101.4) (end 100.579899 101.4) (width 0.2) (layer "F.Cu") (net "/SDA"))
 (segment (start 119.629899 101.4) (end 120.45 100.579899) (width 0.2) (layer "F.Cu") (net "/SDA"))
 (segment (start 105.212116 88.142015) (end 118.470101 101.4) (width 0.2) (layer "F.Cu") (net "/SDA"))
 (segment (start 120.45 94.122861) (end 118.6355 92.308361) (width 0.2) (layer "F.Cu") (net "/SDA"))
 (segment (start 93.025 88.21) (end 93.025 95.004899) (width 0.2) (layer "F.Cu") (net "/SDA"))
 (segment (start 100.579899 101.4) (end 104.0855 97.894399) (width 0.2) (layer "F.Cu") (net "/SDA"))
 (segment (start 101.3855 88.815669) (end 102.059154 88.142015) (width 0.2) (layer "F.Cu") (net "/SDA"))
 (segment (start 118.470101 101.4) (end 119.629899 101.4) (width 0.2) (layer "F.Cu") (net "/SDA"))
 (segment (start 100 87.661169) (end 103.449154 84.212015) (width 0.2) (layer "F.Cu") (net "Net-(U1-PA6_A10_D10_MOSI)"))
 (segment (start 100 100) (end 100 87.661169) (width 0.2) (layer "F.Cu") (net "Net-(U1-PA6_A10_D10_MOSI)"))
 (segment (start 103.449154 84.212015) (end 104.4855 84.212015) (width 0.2) (layer "F.Cu") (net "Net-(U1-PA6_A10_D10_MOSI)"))
 (segment (start 100 119.05) (end 104.4855 114.5645) (width 0.2) (layer "F.Cu") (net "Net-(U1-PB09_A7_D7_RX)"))
 (segment (start 104.4855 114.5645) (end 104.4855 91.832015) (width 0.2) (layer "F.Cu") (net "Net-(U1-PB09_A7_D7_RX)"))
 (segment (start 128.31 82.95) (end 119.437139 82.95) (width 0.2) (layer "F.Cu") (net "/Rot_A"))
 (segment (start 118.6355 77.692015) (end 119.7355 76.592015) (width 0.2) (layer "F.Cu") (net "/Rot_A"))
 (segment (start 119.437139 82.95) (end 118.6355 82.148361) (width 0.2) (layer "F.Cu") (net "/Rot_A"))
 (segment (start 118.6355 82.148361) (end 118.6355 77.692015) (width 0.2) (layer "F.Cu") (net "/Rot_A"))
 (segment (start 140.971522 87.95) (end 142.271522 89.25) (width 0.2) (layer "F.Cu") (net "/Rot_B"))
 (segment (start 143.348478 89.25) (end 144.51 88.088478) (width 0.2) (layer "F.Cu") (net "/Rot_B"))
 (segment (start 128.31 87.95) (end 140.971522 87.95) (width 0.2) (layer "F.Cu") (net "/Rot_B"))
 (segment (start 140.764164 78.5) (end 120.367515 78.5) (width 0.2) (layer "F.Cu") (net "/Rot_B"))
 (segment (start 144.51 88.088478) (end 144.51 82.245836) (width 0.2) (layer "F.Cu") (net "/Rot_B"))
 (segment (start 120.367515 78.5) (end 119.7355 79.132015) (width 0.2) (layer "F.Cu") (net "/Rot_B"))
 (segment (start 144.51 82.245836) (end 140.764164 78.5) (width 0.2) (layer "F.Cu") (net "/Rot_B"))
 (segment (start 142.271522 89.25) (end 143.348478 89.25) (width 0.2) (layer "F.Cu") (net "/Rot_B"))
 (segment (start 144.11 82.411522) (end 143.348478 81.65) (width 0.2) (layer "F.Cu") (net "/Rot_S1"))
 (segment (start 143.348478 81.65) (end 119.757515 81.65) (width 0.2) (layer "F.Cu") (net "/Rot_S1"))
 (segment (start 142.81 87.95) (end 144.11 86.65) (width 0.2) (layer "F.Cu") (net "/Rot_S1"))
 (segment (start 144.11 86.65) (end 144.11 82.411522) (width 0.2) (layer "F.Cu") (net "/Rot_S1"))
 (segment (start 119.757515 81.65) (end 119.7355 81.672015) (width 0.2) (layer "F.Cu") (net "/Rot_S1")))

